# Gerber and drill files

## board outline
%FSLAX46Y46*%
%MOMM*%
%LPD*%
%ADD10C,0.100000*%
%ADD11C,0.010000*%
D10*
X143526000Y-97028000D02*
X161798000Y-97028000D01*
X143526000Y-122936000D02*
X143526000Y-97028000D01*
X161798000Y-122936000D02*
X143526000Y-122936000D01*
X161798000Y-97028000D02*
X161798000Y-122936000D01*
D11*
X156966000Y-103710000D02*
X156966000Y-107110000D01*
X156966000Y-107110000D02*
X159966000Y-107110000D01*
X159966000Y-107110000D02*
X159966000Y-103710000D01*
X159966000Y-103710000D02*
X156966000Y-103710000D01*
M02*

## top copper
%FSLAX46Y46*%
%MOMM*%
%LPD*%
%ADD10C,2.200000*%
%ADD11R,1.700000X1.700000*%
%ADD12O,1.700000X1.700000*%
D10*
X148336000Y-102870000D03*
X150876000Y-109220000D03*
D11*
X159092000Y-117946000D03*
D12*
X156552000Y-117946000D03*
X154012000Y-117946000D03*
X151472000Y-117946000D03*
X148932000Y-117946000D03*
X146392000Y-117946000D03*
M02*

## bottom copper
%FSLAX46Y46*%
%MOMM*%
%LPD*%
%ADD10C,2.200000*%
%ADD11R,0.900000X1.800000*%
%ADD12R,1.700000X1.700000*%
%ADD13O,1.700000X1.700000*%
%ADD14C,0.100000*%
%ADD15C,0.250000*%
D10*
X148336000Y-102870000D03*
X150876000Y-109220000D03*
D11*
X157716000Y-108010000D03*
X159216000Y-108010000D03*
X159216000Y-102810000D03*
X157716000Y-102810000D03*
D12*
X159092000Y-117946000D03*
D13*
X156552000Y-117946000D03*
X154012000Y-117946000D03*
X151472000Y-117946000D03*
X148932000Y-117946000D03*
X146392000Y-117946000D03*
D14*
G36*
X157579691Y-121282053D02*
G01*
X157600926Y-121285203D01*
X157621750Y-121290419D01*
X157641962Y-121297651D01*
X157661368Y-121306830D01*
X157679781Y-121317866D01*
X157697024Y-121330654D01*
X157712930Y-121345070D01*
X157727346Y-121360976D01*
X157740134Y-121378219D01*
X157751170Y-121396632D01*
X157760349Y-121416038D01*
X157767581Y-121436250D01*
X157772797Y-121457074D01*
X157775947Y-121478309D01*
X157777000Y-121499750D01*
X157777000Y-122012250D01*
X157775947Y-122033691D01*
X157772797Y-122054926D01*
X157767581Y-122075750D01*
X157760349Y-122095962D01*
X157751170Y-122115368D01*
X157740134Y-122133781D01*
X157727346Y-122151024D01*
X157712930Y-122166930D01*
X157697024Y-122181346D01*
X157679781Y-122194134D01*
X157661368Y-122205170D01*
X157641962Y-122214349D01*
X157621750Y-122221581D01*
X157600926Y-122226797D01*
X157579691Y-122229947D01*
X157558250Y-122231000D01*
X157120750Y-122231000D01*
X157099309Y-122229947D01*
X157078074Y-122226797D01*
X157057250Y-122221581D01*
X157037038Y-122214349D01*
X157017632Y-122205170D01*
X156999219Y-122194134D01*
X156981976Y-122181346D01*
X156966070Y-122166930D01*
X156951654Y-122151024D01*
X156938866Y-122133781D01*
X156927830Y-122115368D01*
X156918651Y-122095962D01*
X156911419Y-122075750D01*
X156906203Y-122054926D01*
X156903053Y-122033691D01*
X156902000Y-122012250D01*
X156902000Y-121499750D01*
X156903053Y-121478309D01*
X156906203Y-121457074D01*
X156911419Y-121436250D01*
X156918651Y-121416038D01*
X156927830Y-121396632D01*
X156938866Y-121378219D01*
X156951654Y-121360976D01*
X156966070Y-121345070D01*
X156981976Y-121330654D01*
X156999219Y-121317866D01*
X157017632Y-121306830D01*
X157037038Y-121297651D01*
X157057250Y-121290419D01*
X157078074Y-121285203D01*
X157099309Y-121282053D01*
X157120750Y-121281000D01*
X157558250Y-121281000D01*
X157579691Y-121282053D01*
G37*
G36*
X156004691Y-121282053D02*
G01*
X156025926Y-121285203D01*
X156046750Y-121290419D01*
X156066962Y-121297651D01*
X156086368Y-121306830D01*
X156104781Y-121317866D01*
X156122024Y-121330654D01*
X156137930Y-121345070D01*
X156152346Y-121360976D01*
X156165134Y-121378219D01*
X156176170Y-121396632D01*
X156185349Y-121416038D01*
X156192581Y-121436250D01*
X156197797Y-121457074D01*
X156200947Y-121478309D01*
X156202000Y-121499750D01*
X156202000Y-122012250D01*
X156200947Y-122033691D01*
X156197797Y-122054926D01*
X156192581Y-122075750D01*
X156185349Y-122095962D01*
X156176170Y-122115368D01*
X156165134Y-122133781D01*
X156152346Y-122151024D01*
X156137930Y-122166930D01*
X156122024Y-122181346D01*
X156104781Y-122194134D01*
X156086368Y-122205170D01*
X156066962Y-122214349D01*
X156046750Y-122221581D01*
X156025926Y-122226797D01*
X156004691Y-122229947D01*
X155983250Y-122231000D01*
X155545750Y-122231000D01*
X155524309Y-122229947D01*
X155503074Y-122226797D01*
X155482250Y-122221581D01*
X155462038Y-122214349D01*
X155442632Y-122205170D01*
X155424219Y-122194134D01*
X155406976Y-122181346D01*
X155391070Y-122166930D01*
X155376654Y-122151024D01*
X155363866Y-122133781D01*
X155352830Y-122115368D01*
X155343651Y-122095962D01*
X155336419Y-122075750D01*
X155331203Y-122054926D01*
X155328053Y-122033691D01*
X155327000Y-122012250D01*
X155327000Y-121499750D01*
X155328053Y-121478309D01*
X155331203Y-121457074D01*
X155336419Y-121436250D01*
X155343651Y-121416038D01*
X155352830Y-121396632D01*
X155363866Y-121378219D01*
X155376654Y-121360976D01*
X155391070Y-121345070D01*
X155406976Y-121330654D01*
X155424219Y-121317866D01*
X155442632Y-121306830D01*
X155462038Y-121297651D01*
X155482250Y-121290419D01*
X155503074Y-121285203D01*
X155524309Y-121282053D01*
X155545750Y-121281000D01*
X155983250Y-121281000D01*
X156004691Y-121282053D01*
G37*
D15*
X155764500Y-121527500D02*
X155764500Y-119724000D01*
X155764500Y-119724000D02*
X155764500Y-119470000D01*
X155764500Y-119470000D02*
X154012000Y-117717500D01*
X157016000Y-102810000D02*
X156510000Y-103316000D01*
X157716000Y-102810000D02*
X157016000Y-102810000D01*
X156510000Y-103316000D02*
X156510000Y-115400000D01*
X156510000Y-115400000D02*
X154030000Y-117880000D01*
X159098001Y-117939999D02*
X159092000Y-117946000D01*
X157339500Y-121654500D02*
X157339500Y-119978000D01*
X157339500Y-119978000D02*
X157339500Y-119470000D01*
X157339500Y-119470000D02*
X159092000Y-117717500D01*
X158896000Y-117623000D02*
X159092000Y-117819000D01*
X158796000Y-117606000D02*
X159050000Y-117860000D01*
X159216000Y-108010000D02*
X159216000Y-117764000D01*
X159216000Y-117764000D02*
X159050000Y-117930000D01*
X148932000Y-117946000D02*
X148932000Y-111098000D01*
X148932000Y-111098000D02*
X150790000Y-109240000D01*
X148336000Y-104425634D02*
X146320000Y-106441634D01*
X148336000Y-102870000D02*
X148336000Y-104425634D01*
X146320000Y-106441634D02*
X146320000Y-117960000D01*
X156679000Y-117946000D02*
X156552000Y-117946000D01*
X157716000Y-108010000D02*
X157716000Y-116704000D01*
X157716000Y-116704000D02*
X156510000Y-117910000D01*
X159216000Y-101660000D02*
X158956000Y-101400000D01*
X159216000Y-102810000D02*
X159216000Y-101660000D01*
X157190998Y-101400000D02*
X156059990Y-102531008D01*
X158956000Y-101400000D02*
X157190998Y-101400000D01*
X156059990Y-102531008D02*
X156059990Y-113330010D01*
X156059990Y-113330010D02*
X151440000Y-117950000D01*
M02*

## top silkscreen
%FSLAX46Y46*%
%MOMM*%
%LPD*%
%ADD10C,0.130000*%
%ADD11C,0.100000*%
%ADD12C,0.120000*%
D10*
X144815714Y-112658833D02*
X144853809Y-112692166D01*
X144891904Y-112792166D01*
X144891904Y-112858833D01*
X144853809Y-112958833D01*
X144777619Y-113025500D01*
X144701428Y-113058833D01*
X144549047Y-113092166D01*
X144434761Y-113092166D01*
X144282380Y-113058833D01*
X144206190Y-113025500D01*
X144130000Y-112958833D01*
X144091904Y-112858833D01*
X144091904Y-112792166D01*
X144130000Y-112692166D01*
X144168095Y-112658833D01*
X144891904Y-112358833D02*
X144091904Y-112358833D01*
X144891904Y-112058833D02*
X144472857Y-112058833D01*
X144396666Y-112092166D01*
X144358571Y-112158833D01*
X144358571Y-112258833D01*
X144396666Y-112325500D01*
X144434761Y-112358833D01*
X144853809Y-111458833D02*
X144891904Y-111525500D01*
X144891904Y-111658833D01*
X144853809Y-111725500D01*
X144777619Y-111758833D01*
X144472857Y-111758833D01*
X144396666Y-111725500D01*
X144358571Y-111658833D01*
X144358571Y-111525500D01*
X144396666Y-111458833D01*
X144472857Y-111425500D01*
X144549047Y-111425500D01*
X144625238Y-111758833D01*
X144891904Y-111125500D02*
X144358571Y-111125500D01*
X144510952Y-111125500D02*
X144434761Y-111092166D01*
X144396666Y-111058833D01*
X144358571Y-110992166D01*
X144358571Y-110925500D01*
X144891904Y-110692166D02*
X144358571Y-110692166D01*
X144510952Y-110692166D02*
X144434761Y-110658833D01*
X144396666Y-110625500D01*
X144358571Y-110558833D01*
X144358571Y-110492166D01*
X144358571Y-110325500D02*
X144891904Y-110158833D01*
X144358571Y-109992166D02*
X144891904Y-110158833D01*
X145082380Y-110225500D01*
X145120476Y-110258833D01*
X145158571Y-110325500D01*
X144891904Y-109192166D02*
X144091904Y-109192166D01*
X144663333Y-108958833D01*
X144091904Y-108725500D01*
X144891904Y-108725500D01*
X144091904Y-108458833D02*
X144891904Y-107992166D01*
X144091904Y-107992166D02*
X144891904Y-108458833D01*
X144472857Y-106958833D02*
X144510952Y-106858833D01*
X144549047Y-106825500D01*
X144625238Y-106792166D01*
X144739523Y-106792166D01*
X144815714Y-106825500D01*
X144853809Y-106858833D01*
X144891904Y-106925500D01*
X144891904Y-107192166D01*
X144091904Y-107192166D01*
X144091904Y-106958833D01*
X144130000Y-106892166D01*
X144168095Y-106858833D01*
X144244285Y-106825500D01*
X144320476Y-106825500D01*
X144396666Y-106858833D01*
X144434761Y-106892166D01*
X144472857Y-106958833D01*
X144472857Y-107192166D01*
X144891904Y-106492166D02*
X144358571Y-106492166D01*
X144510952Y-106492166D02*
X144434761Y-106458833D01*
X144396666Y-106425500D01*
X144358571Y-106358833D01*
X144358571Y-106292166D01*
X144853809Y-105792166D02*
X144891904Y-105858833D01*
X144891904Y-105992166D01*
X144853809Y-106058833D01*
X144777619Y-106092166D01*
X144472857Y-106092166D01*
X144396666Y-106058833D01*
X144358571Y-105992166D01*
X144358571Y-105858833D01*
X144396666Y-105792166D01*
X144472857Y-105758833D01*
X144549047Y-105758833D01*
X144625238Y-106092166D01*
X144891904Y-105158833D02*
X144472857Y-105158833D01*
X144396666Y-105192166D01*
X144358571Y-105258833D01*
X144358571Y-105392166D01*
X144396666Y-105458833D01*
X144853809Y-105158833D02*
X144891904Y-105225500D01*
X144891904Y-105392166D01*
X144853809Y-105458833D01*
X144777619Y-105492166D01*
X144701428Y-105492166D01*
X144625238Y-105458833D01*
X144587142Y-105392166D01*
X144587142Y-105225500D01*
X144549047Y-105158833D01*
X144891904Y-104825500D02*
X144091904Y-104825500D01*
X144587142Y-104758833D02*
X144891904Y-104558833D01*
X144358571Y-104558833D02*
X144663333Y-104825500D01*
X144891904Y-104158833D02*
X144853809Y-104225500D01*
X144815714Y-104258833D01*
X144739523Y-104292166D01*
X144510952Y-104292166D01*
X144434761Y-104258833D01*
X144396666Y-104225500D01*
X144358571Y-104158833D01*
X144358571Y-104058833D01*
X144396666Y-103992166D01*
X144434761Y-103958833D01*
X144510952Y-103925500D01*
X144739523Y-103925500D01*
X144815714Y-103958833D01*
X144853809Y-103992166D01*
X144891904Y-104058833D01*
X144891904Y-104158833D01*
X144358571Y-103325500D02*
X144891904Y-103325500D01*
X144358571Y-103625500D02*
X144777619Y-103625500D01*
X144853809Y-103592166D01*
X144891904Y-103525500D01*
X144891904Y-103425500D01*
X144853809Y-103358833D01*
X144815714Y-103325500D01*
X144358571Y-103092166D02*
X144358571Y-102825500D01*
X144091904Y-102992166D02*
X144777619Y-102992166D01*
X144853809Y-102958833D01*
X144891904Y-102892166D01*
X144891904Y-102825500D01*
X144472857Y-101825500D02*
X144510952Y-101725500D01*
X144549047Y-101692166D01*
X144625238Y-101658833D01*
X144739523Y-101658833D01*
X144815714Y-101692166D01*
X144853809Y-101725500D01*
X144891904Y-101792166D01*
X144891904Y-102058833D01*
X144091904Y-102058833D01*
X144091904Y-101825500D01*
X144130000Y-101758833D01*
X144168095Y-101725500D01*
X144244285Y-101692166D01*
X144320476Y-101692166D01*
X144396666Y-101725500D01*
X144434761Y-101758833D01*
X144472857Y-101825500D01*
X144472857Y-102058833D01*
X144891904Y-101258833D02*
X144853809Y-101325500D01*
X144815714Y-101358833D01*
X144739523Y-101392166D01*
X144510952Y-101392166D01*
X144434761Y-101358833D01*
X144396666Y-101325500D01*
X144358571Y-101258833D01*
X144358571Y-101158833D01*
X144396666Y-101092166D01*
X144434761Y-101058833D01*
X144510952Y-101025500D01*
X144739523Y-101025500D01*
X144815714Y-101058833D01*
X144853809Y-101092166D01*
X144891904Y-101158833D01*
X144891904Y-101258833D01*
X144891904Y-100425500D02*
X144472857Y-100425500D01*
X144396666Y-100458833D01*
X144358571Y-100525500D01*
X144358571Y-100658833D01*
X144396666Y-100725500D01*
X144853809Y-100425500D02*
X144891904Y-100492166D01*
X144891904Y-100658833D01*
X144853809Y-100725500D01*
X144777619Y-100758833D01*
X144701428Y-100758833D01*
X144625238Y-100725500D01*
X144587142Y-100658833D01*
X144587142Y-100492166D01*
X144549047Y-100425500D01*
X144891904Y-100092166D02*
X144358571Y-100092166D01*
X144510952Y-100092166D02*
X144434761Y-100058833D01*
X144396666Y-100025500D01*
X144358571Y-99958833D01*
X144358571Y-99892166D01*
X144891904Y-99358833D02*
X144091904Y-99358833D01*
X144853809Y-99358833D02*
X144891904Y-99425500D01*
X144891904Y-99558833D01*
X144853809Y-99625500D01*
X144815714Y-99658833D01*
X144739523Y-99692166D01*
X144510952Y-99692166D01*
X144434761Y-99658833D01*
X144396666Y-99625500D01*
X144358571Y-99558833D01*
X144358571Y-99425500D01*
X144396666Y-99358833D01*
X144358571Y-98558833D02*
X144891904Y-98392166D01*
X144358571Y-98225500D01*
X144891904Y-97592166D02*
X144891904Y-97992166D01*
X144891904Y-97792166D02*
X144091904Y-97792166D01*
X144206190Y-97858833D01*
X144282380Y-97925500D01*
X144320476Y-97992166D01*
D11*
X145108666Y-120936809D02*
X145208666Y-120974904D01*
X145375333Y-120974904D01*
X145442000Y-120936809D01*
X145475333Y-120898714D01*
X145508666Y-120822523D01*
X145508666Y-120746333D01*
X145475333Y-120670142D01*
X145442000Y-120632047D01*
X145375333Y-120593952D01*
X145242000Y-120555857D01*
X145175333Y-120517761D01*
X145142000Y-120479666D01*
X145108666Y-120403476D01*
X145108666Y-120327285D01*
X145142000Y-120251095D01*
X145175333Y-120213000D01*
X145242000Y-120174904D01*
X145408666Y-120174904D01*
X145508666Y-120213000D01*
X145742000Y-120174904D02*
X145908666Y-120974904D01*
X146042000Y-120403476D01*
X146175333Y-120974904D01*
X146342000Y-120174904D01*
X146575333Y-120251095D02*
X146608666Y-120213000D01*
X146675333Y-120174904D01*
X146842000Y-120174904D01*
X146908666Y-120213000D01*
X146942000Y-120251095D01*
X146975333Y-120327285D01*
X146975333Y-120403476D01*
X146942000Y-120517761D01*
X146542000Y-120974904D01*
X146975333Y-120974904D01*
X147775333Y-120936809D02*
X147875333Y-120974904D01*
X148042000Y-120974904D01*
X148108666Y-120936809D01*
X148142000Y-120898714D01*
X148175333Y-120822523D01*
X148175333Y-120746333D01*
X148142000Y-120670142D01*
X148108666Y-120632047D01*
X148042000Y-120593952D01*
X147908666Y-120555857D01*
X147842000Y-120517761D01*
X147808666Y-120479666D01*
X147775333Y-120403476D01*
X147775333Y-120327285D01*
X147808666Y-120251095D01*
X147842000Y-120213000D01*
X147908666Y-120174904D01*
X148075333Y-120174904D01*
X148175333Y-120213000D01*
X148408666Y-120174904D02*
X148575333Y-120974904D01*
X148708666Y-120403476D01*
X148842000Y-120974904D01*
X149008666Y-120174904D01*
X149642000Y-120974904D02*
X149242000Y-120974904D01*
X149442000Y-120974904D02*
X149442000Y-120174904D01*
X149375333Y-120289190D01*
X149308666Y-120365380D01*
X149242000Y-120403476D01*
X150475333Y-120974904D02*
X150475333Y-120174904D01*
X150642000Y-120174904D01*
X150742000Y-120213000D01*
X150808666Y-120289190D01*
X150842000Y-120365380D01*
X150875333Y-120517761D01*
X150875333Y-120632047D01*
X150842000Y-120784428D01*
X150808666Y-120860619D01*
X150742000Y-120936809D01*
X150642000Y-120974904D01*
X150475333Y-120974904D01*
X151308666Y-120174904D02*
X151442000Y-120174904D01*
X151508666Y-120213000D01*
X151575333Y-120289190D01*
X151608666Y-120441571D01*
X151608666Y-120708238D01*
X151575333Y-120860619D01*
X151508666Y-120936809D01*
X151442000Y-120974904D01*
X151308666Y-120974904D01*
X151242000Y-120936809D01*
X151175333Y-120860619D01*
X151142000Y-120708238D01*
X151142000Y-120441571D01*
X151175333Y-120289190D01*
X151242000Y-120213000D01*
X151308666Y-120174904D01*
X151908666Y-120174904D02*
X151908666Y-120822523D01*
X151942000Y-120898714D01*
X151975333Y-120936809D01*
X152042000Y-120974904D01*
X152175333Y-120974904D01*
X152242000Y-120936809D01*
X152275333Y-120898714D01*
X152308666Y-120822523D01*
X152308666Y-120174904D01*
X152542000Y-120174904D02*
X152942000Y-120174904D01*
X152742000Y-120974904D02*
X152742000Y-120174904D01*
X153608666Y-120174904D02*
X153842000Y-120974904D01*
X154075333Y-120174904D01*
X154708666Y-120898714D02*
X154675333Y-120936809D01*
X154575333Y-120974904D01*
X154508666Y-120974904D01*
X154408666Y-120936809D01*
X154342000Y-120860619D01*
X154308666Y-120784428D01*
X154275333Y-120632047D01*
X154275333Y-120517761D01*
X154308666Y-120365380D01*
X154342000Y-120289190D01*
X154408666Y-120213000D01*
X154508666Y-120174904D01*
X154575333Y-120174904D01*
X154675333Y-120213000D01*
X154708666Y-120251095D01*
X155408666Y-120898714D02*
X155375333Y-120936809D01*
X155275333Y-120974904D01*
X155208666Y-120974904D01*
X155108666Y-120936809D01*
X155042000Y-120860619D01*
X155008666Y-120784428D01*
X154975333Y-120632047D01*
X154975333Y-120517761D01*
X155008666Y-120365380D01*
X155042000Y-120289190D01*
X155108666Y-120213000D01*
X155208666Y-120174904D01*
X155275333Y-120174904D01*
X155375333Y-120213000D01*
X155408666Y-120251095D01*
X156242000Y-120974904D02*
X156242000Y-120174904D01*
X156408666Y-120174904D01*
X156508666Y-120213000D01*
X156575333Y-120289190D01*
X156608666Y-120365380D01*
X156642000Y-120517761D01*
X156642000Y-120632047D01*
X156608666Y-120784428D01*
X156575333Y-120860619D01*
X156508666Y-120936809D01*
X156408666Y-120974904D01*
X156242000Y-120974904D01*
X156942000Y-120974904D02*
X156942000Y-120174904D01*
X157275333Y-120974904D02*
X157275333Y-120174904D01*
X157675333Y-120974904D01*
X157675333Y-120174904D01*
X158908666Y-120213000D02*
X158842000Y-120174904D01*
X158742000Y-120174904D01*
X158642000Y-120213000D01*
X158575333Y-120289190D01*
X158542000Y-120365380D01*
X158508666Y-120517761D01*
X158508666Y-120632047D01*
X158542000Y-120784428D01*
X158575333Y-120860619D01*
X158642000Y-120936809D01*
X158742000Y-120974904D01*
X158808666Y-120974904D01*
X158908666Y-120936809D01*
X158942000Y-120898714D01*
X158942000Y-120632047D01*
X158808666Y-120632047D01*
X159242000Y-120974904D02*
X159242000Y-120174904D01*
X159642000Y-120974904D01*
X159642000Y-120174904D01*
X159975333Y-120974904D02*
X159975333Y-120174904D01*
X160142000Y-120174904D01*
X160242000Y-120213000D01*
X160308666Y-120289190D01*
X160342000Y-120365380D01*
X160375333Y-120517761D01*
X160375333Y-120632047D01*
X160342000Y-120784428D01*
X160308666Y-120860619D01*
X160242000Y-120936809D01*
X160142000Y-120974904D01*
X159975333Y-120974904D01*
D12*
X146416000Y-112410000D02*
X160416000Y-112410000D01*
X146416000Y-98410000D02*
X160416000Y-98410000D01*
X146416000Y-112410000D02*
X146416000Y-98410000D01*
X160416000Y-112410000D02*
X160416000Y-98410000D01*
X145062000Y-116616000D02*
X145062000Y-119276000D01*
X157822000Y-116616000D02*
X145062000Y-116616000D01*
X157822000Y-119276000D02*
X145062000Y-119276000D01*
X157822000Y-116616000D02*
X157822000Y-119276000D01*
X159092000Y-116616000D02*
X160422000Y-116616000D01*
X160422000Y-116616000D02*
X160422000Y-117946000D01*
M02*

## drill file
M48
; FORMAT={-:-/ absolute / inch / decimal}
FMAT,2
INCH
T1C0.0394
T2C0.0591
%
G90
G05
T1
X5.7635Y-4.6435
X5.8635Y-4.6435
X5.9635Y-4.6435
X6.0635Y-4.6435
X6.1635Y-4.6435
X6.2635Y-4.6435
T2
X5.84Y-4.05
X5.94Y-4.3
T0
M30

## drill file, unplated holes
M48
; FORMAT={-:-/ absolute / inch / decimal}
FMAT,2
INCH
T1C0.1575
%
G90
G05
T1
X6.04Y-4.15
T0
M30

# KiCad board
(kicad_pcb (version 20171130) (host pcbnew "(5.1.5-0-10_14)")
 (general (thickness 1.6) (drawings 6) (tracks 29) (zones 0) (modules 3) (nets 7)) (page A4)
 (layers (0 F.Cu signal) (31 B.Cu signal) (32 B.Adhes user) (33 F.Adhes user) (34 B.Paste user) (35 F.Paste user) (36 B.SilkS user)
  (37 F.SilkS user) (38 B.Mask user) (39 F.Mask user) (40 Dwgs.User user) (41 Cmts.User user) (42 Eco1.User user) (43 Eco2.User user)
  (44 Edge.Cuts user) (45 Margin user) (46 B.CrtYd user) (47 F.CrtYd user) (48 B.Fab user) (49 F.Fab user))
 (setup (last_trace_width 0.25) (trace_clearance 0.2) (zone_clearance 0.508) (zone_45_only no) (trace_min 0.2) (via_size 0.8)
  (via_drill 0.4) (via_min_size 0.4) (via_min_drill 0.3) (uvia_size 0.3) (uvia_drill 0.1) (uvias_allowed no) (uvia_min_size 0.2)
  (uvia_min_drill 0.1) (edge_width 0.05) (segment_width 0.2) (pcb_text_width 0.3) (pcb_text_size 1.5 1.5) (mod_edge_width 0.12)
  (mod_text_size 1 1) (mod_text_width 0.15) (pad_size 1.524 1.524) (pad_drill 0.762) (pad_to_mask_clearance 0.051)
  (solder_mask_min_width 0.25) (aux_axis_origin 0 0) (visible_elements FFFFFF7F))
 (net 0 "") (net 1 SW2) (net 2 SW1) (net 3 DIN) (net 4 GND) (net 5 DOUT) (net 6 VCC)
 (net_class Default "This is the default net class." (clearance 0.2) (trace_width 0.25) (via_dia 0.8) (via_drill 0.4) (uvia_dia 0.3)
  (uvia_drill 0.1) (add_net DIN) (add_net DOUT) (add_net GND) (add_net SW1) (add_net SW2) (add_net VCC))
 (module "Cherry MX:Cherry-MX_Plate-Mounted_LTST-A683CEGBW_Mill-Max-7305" (layer F.Cu) (at 153.416 105.41 90)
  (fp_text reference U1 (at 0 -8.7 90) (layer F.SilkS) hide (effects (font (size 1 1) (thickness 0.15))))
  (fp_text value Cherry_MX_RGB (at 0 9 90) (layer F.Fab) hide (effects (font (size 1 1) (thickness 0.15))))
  (fp_poly (pts (xy 1.7 3.55) (xy -1.7 3.55) (xy -1.7 6.55) (xy 1.7 6.55)) (layer Edge.Cuts) (width 0.01))
  (fp_line (start -7 -7) (end -7 7) (layer F.SilkS) (width 0.12))
  (fp_line (start 7 -7) (end 7 7) (layer F.SilkS) (width 0.12))
  (fp_line (start -7 -7) (end 7 -7) (layer F.SilkS) (width 0.12))
  (fp_line (start -7 7) (end 7 7) (layer F.SilkS) (width 0.12))
  (pad "" np_thru_hole circle (at 0 0 90) (size 4 4) (drill 4) (layers *.Cu *.Mask))
  (pad 6 thru_hole circle (at 2.54 -5.08 90) (size 2.2 2.2) (drill 1.5) (layers *.Cu *.Mask) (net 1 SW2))
  (pad 5 thru_hole circle (at -3.81 -2.54 90) (size 2.2 2.2) (drill 1.5) (layers *.Cu *.Mask) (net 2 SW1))
  (pad 2 smd rect (at -2.6 4.3 90) (size 1.8 0.9) (layers B.Cu B.Paste B.Mask) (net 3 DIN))
  (pad 1 smd rect (at -2.6 5.8 90) (size 1.8 0.9) (layers B.Cu B.Paste B.Mask) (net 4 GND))
  (pad 3 smd rect (at 2.6 5.8 90) (size 1.8 0.9) (layers B.Cu B.Paste B.Mask) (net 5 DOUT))
  (pad 4 smd rect (at 2.6 4.3 90) (size 1.8 0.9) (layers B.Cu B.Paste B.Mask) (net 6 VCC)))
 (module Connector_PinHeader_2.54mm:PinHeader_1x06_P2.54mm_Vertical (layer F.Cu) (at 159.092 117.946 270)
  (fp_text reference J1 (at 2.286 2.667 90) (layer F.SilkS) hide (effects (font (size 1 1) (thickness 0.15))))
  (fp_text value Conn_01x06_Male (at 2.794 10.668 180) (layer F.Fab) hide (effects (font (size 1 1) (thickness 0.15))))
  (fp_line (start -1.33 14.03) (end 1.33 14.03) (layer F.SilkS) (width 0.12))
  (fp_line (start -1.33 1.27) (end -1.33 14.03) (layer F.SilkS) (width 0.12))
  (fp_line (start 1.33 1.27) (end 1.33 14.03) (layer F.SilkS) (width 0.12))
  (fp_line (start -1.33 1.27) (end 1.33 1.27) (layer F.SilkS) (width 0.12))
  (fp_line (start -1.33 0) (end -1.33 -1.33) (layer F.SilkS) (width 0.12))
  (fp_line (start -1.33 -1.33) (end 0 -1.33) (layer F.SilkS) (width 0.12))
  (pad 1 thru_hole rect (at 0 0 270) (size 1.7 1.7) (drill 1) (layers *.Cu *.Mask) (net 4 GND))
  (pad 2 thru_hole oval (at 0 2.54 270) (size 1.7 1.7) (drill 1) (layers *.Cu *.Mask) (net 3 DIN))
  (pad 3 thru_hole oval (at 0 5.08 270) (size 1.7 1.7) (drill 1) (layers *.Cu *.Mask) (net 6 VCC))
  (pad 4 thru_hole oval (at 0 7.62 270) (size 1.7 1.7) (drill 1) (layers *.Cu *.Mask) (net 5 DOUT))
  (pad 5 thru_hole oval (at 0 10.16 270) (size 1.7 1.7) (drill 1) (layers *.Cu *.Mask) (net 2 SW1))
  (pad 6 thru_hole oval (at 0 12.7 270) (size 1.7 1.7) (drill 1) (layers *.Cu *.Mask) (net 1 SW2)))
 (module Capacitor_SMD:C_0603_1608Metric (layer B.Cu) (at 156.552 121.756)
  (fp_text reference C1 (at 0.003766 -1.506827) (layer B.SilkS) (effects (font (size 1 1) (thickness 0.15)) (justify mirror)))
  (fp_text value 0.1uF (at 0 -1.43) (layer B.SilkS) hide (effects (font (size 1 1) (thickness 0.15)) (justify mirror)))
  (pad 2 smd roundrect (at 0.7875 0) (size 0.875 0.95) (layers B.Cu B.Paste B.Mask) (roundrect_rratio 0.25) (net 4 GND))
  (pad 1 smd roundrect (at -0.7875 0) (size 0.875 0.95) (layers B.Cu B.Paste B.Mask) (roundrect_rratio 0.25) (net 6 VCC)))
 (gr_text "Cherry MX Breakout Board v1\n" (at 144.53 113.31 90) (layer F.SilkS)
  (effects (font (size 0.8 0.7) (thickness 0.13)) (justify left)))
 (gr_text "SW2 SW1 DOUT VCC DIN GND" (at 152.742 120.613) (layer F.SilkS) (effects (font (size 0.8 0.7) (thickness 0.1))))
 (gr_line (start 143.526 97.028) (end 161.798 97.028) (layer Edge.Cuts) (width 0.1))
 (gr_line (start 143.526 122.936) (end 143.526 97.028) (layer Edge.Cuts) (width 0.1))
 (gr_line (start 161.798 122.936) (end 143.526 122.936) (layer Edge.Cuts) (width 0.1))
 (gr_line (start 161.798 97.028) (end 161.798 122.936) (layer Edge.Cuts) (width 0.1))
 (segment (start 155.7645 121.5275) (end 155.7645 119.724) (width 0.25) (layer B.Cu) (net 6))
 (segment (start 155.7645 119.724) (end 155.7645 119.47) (width 0.25) (layer B.Cu) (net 6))
 (segment (start 155.7645 119.47) (end 154.012 117.7175) (width 0.25) (layer B.Cu) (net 6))
 (segment (start 157.016 102.81) (end 156.51 103.316) (width 0.25) (layer B.Cu) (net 6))
 (segment (start 157.716 102.81) (end 157.016 102.81) (width 0.25) (layer B.Cu) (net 6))
 (segment (start 156.51 103.316) (end 156.51 115.4) (width 0.25) (layer B.Cu) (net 6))
 (segment (start 156.51 115.4) (end 154.03 117.88) (width 0.25) (layer B.Cu) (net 6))
 (segment (start 159.098001 117.939999) (end 159.092 117.946) (width 0.25) (layer B.Cu) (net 4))
 (segment (start 157.3395 121.6545) (end 157.3395 119.978) (width 0.25) (layer B.Cu) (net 4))
 (segment (start 157.3395 119.978) (end 157.3395 119.47) (width 0.25) (layer B.Cu) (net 4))
 (segment (start 157.3395 119.47) (end 159.092 117.7175) (width 0.25) (layer B.Cu) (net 4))
 (segment (start 158.896 117.623) (end 159.092 117.819) (width 0.25) (layer B.Cu) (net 4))
 (segment (start 158.796 117.606) (end 159.05 117.86) (width 0.25) (layer B.Cu) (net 4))
 (segment (start 159.216 108.01) (end 159.216 117.764) (width 0.25) (layer B.Cu) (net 4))
 (segment (start 159.216 117.764) (end 159.05 117.93) (width 0.25) (layer B.Cu) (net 4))
 (segment (start 148.932 117.946) (end 148.932 111.098) (width 0.25) (layer B.Cu) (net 2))
 (segment (start 148.932 111.098) (end 150.79 109.24) (width 0.25) (layer B.Cu) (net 2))
 (segment (start 148.336 104.425634) (end 146.32 106.441634) (width 0.25) (layer B.Cu) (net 1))
 (segment (start 148.336 102.87) (end 148.336 104.425634) (width 0.25) (layer B.Cu) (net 1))
 (segment (start 146.32 106.441634) (end 146.32 117.96) (width 0.25) (layer B.Cu) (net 1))
 (segment (start 156.679 117.946) (end 156.552 117.946) (width 0.25) (layer B.Cu) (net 3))
 (segment (start 157.716 108.01) (end 157.716 116.704) (width 0.25) (layer B.Cu) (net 3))
 (segment (start 157.716 116.704) (end 156.51 117.91) (width 0.25) (layer B.Cu) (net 3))
 (segment (start 159.216 101.66) (end 158.956 101.4) (width 0.25) (layer B.Cu) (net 5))
 (segment (start 159.216 102.81) (end 159.216 101.66) (width 0.25) (layer B.Cu) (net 5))
 (segment (start 157.190998 101.4) (end 156.05999 102.531008) (width 0.25) (layer B.Cu) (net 5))
 (segment (start 158.956 101.4) (end 157.190998 101.4) (width 0.25) (layer B.Cu) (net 5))
 (segment (start 156.05999 102.531008) (end 156.05999 113.33001) (width 0.25) (layer B.Cu) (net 5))
 (segment (start 156.05999 113.33001) (end 151.44 117.95) (width 0.25) (layer B.Cu) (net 5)))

